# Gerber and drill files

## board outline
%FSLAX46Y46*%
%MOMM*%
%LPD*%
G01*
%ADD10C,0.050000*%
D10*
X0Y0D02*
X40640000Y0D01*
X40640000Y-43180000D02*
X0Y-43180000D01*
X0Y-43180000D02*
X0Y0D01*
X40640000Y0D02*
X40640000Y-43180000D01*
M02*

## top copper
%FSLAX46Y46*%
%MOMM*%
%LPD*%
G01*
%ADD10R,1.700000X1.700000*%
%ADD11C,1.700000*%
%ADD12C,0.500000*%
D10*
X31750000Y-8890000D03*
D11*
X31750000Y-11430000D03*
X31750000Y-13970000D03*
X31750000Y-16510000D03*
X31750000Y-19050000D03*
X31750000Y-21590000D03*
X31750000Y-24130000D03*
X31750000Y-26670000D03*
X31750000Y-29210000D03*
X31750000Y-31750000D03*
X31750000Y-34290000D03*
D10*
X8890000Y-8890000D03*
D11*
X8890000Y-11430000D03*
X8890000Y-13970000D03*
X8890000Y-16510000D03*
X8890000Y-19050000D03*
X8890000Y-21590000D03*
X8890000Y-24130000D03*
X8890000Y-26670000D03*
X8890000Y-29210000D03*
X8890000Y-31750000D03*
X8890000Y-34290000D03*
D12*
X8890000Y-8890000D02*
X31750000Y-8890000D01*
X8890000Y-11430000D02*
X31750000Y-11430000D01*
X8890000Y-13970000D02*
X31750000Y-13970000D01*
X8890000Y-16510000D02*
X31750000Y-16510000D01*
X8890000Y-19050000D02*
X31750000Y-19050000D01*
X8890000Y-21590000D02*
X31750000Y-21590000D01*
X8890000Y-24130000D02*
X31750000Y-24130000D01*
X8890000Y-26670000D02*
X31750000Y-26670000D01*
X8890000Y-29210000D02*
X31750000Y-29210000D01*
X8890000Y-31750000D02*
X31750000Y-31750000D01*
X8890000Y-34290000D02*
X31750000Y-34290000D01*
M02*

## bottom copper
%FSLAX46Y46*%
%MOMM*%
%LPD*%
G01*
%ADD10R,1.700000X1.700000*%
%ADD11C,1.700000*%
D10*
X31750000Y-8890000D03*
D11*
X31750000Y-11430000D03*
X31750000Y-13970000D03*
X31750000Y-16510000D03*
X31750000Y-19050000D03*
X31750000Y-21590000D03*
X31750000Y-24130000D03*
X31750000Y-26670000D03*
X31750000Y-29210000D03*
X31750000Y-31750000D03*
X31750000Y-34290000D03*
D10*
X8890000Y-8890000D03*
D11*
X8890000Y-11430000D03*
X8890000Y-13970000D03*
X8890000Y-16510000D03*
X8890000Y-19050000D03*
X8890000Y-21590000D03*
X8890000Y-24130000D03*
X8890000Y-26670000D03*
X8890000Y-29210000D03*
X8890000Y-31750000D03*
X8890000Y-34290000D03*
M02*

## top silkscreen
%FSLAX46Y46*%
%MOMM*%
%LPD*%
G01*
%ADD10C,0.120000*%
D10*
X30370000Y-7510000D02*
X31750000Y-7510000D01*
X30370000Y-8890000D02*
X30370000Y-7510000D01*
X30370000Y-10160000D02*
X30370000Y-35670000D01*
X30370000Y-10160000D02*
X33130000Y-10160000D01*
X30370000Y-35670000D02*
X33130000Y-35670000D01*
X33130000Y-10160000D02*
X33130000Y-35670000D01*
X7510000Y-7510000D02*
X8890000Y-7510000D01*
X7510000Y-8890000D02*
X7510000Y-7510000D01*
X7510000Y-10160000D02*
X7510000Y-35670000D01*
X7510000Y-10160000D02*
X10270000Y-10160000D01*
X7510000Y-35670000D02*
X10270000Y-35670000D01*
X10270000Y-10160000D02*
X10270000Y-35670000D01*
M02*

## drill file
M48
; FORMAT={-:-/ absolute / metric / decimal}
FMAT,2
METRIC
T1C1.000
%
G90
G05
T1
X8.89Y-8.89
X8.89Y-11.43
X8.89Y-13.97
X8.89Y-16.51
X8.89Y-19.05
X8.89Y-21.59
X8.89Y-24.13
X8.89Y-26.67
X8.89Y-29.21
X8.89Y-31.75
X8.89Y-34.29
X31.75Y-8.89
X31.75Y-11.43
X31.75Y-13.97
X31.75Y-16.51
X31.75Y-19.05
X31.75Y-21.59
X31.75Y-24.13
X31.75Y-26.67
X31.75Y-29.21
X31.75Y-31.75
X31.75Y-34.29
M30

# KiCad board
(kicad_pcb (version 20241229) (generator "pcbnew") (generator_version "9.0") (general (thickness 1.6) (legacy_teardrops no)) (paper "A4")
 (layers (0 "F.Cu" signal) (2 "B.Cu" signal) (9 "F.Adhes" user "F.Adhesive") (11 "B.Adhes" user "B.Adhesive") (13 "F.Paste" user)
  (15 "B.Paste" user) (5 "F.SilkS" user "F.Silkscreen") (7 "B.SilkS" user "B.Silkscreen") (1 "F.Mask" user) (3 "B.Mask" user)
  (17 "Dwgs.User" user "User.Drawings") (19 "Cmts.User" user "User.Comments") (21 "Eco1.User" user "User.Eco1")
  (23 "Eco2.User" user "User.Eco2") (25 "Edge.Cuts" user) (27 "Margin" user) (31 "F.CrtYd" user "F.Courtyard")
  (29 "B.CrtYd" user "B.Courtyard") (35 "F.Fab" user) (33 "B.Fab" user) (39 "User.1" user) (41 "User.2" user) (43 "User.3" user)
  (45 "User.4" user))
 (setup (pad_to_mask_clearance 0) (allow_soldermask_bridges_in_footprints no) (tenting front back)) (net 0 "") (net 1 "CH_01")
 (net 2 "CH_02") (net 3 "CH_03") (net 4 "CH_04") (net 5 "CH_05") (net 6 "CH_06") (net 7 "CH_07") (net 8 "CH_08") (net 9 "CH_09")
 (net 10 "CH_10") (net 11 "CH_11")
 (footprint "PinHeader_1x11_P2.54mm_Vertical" (layer "F.Cu") (at 31.75 8.89)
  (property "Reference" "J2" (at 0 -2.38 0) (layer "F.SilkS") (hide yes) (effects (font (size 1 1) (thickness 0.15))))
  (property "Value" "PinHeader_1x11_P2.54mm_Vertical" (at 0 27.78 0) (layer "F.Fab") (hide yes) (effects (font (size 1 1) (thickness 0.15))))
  (fp_line (start -1.38 -1.38) (end 0 -1.38) (stroke (width 0.12) (type solid)) (layer "F.SilkS"))
  (fp_line (start -1.38 0) (end -1.38 -1.38) (stroke (width 0.12) (type solid)) (layer "F.SilkS"))
  (fp_line (start -1.38 1.27) (end -1.38 26.78) (stroke (width 0.12) (type solid)) (layer "F.SilkS"))
  (fp_line (start -1.38 1.27) (end 1.38 1.27) (stroke (width 0.12) (type solid)) (layer "F.SilkS"))
  (fp_line (start -1.38 26.78) (end 1.38 26.78) (stroke (width 0.12) (type solid)) (layer "F.SilkS"))
  (fp_line (start 1.38 1.27) (end 1.38 26.78) (stroke (width 0.12) (type solid)) (layer "F.SilkS"))
  (pad "1" thru_hole rect (at 0 0) (size 1.7 1.7) (drill 1) (layers "*.Cu" "*.Mask") (remove_unused_layers no) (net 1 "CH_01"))
  (pad "2" thru_hole circle (at 0 2.54) (size 1.7 1.7) (drill 1) (layers "*.Cu" "*.Mask") (remove_unused_layers no) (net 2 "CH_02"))
  (pad "3" thru_hole circle (at 0 5.08) (size 1.7 1.7) (drill 1) (layers "*.Cu" "*.Mask") (remove_unused_layers no) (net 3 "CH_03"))
  (pad "4" thru_hole circle (at 0 7.62) (size 1.7 1.7) (drill 1) (layers "*.Cu" "*.Mask") (remove_unused_layers no) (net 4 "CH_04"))
  (pad "5" thru_hole circle (at 0 10.16) (size 1.7 1.7) (drill 1) (layers "*.Cu" "*.Mask") (remove_unused_layers no) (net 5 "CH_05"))
  (pad "6" thru_hole circle (at 0 12.7) (size 1.7 1.7) (drill 1) (layers "*.Cu" "*.Mask") (remove_unused_layers no) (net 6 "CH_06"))
  (pad "7" thru_hole circle (at 0 15.24) (size 1.7 1.7) (drill 1) (layers "*.Cu" "*.Mask") (remove_unused_layers no) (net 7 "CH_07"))
  (pad "8" thru_hole circle (at 0 17.78) (size 1.7 1.7) (drill 1) (layers "*.Cu" "*.Mask") (remove_unused_layers no) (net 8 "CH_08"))
  (pad "9" thru_hole circle (at 0 20.32) (size 1.7 1.7) (drill 1) (layers "*.Cu" "*.Mask") (remove_unused_layers no) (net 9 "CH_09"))
  (pad "10" thru_hole circle (at 0 22.86) (size 1.7 1.7) (drill 1) (layers "*.Cu" "*.Mask") (remove_unused_layers no) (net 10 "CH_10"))
  (pad "11" thru_hole circle (at 0 25.4) (size 1.7 1.7) (drill 1) (layers "*.Cu" "*.Mask") (remove_unused_layers no) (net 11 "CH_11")))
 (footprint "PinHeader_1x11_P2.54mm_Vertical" (layer "F.Cu") (at 8.89 8.89)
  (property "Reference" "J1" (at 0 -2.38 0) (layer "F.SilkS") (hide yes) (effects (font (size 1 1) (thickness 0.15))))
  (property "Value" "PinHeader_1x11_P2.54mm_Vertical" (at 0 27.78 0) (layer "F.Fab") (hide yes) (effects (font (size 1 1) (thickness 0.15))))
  (fp_line (start -1.38 -1.38) (end 0 -1.38) (stroke (width 0.12) (type solid)) (layer "F.SilkS"))
  (fp_line (start -1.38 0) (end -1.38 -1.38) (stroke (width 0.12) (type solid)) (layer "F.SilkS"))
  (fp_line (start -1.38 1.27) (end -1.38 26.78) (stroke (width 0.12) (type solid)) (layer "F.SilkS"))
  (fp_line (start -1.38 1.27) (end 1.38 1.27) (stroke (width 0.12) (type solid)) (layer "F.SilkS"))
  (fp_line (start -1.38 26.78) (end 1.38 26.78) (stroke (width 0.12) (type solid)) (layer "F.SilkS"))
  (fp_line (start 1.38 1.27) (end 1.38 26.78) (stroke (width 0.12) (type solid)) (layer "F.SilkS"))
  (pad "1" thru_hole rect (at 0 0) (size 1.7 1.7) (drill 1) (layers "*.Cu" "*.Mask") (remove_unused_layers no) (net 1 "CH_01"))
  (pad "2" thru_hole circle (at 0 2.54) (size 1.7 1.7) (drill 1) (layers "*.Cu" "*.Mask") (remove_unused_layers no) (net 2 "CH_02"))
  (pad "3" thru_hole circle (at 0 5.08) (size 1.7 1.7) (drill 1) (layers "*.Cu" "*.Mask") (remove_unused_layers no) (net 3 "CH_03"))
  (pad "4" thru_hole circle (at 0 7.62) (size 1.7 1.7) (drill 1) (layers "*.Cu" "*.Mask") (remove_unused_layers no) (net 4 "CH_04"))
  (pad "5" thru_hole circle (at 0 10.16) (size 1.7 1.7) (drill 1) (layers "*.Cu" "*.Mask") (remove_unused_layers no) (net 5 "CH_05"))
  (pad "6" thru_hole circle (at 0 12.7) (size 1.7 1.7) (drill 1) (layers "*.Cu" "*.Mask") (remove_unused_layers no) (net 6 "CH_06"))
  (pad "7" thru_hole circle (at 0 15.24) (size 1.7 1.7) (drill 1) (layers "*.Cu" "*.Mask") (remove_unused_layers no) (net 7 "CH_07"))
  (pad "8" thru_hole circle (at 0 17.78) (size 1.7 1.7) (drill 1) (layers "*.Cu" "*.Mask") (remove_unused_layers no) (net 8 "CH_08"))
  (pad "9" thru_hole circle (at 0 20.32) (size 1.7 1.7) (drill 1) (layers "*.Cu" "*.Mask") (remove_unused_layers no) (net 9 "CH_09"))
  (pad "10" thru_hole circle (at 0 22.86) (size 1.7 1.7) (drill 1) (layers "*.Cu" "*.Mask") (remove_unused_layers no) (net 10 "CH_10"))
  (pad "11" thru_hole circle (at 0 25.4) (size 1.7 1.7) (drill 1) (layers "*.Cu" "*.Mask") (remove_unused_layers no) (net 11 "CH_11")))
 (gr_line (start 0 0) (end 40.64 0) (stroke (width 0.05) (type default)) (layer "Edge.Cuts"))
 (gr_line (start 40.64 43.18) (end 0 43.18) (stroke (width 0.05) (type default)) (layer "Edge.Cuts"))
 (gr_line (start 0 43.18) (end 0 0) (stroke (width 0.05) (type default)) (layer "Edge.Cuts"))
 (gr_line (start 40.64 0) (end 40.64 43.18) (stroke (width 0.05) (type default)) (layer "Edge.Cuts"))
 (segment (start 8.89 8.89) (end 31.75 8.89) (width 0.5) (layer "F.Cu") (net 1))
 (segment (start 8.89 11.43) (end 31.75 11.43) (width 0.5) (layer "F.Cu") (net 2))
 (segment (start 8.89 13.97) (end 31.75 13.97) (width 0.5) (layer "F.Cu") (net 3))
 (segment (start 8.89 16.51) (end 31.75 16.51) (width 0.5) (layer "F.Cu") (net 4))
 (segment (start 8.89 19.05) (end 31.75 19.05) (width 0.5) (layer "F.Cu") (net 5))
 (segment (start 8.89 21.59) (end 31.75 21.59) (width 0.5) (layer "F.Cu") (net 6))
 (segment (start 8.89 24.13) (end 31.75 24.13) (width 0.5) (layer "F.Cu") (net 7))
 (segment (start 8.89 26.67) (end 31.75 26.67) (width 0.5) (layer "F.Cu") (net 8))
 (segment (start 8.89 29.21) (end 31.75 29.21) (width 0.5) (layer "F.Cu") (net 9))
 (segment (start 8.89 31.75) (end 31.75 31.75) (width 0.5) (layer "F.Cu") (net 10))
 (segment (start 8.89 34.29) (end 31.75 34.29) (width 0.5) (layer "F.Cu") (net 11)))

